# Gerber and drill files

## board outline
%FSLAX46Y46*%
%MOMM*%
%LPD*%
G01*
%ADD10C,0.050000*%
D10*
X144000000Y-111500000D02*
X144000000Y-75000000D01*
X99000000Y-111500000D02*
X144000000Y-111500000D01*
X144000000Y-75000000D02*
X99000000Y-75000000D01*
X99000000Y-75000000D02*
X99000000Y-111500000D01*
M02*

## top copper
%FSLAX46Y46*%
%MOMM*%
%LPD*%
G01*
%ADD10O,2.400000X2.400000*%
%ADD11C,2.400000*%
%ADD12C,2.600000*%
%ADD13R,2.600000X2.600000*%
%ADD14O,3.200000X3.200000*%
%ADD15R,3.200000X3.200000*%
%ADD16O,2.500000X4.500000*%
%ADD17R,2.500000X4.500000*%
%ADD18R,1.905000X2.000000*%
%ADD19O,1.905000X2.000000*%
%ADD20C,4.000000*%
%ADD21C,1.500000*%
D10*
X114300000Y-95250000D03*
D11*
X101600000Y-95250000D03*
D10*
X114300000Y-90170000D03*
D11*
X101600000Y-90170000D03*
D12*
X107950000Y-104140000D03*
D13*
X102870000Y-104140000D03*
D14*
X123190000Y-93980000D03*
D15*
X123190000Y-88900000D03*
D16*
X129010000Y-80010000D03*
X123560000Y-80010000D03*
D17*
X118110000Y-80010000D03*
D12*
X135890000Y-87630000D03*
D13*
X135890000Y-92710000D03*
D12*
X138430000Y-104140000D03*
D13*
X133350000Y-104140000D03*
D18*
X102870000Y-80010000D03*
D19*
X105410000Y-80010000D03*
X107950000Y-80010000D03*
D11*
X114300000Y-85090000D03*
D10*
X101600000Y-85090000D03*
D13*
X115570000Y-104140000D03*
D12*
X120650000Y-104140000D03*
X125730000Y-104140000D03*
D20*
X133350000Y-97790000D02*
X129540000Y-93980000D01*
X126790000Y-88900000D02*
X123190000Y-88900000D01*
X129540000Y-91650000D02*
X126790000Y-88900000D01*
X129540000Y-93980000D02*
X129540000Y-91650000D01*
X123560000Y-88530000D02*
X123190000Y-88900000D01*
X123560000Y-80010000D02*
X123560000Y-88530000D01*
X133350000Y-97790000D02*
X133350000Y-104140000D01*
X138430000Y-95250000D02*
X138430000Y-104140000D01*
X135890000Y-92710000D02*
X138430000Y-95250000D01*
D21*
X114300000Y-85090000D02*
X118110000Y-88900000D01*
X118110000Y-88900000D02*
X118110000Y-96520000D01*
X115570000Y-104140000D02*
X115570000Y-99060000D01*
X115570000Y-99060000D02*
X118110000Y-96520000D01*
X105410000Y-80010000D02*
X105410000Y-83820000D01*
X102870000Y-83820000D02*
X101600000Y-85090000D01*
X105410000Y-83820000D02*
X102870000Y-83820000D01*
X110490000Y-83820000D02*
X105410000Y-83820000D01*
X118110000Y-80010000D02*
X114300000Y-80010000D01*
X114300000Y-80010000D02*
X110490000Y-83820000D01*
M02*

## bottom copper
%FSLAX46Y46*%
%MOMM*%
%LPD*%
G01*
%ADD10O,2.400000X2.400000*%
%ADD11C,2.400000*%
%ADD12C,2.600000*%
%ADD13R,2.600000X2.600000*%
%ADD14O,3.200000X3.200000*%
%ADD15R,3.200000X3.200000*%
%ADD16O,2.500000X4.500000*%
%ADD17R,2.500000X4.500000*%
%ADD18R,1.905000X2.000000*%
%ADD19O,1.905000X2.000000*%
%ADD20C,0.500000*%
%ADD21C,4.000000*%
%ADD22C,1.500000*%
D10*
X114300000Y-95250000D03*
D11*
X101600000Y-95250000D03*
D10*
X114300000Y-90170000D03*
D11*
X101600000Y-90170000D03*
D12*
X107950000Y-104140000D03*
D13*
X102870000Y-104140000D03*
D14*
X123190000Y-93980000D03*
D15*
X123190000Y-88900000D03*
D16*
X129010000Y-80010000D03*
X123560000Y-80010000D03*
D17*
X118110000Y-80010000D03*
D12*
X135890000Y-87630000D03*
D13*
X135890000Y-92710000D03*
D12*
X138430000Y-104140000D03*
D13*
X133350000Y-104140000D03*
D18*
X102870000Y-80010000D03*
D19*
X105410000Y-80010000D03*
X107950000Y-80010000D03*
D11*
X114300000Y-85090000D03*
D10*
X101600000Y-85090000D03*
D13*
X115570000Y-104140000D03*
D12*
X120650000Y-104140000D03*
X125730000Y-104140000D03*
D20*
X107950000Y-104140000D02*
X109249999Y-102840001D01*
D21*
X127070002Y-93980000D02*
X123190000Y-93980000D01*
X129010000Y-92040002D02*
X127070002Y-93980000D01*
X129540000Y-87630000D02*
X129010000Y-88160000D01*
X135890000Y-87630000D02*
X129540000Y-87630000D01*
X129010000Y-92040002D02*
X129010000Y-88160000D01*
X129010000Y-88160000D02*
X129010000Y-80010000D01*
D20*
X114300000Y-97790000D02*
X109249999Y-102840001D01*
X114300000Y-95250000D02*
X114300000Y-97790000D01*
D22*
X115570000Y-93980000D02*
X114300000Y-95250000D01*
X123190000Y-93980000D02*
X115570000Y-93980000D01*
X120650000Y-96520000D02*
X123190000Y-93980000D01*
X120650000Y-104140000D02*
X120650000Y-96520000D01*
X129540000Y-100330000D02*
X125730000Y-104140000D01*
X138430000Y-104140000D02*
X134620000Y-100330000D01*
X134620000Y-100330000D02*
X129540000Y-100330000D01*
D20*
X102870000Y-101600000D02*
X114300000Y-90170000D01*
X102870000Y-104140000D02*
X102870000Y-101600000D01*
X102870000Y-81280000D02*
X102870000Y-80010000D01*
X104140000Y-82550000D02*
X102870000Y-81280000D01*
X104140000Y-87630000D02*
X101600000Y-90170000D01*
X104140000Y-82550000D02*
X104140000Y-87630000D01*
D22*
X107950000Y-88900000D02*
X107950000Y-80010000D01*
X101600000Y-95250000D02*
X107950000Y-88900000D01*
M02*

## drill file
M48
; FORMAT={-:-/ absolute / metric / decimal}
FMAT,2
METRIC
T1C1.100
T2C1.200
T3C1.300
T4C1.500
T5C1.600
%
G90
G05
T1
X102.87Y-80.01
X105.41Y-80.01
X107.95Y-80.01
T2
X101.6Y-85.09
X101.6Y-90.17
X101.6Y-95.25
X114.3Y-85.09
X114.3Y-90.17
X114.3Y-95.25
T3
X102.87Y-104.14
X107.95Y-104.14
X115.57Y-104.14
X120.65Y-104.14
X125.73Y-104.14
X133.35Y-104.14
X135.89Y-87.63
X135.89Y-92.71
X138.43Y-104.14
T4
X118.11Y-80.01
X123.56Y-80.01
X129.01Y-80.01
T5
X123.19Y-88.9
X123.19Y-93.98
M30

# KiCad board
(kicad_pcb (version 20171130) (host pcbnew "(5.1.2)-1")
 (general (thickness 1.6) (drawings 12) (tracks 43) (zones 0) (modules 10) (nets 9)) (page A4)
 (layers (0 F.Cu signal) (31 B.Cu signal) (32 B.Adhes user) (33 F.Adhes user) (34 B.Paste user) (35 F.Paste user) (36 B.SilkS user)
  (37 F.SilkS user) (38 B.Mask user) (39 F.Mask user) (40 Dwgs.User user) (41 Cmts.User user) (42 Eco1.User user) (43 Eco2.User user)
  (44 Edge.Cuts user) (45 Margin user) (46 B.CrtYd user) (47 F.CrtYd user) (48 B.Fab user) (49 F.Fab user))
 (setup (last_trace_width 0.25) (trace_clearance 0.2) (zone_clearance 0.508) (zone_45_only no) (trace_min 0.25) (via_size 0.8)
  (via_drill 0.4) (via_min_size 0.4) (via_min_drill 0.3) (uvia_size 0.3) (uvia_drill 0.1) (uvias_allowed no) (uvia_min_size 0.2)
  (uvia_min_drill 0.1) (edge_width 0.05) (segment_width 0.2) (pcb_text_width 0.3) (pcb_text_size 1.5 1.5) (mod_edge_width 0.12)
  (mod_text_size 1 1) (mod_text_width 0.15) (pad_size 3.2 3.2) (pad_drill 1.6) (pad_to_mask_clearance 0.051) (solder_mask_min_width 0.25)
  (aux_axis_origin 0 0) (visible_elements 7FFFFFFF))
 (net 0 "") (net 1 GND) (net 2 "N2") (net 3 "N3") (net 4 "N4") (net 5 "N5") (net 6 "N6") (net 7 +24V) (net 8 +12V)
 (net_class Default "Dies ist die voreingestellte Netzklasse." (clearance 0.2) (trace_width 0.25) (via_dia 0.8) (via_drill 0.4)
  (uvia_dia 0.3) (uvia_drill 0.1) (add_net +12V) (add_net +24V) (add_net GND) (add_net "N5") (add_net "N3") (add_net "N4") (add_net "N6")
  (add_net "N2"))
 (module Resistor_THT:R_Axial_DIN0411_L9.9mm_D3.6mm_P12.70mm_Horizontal (layer F.Cu) (at 101.6 95.25)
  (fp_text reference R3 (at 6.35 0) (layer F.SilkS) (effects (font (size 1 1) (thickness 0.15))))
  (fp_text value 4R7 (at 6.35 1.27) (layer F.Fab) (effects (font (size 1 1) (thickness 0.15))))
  (pad 2 thru_hole oval (at 12.7 0) (size 2.4 2.4) (drill 1.2) (layers *.Cu *.Mask) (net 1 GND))
  (pad 1 thru_hole circle (at 0 0) (size 2.4 2.4) (drill 1.2) (layers *.Cu *.Mask) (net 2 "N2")))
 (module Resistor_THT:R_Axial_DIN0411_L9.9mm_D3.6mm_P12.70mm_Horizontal (layer F.Cu) (at 101.6 90.17)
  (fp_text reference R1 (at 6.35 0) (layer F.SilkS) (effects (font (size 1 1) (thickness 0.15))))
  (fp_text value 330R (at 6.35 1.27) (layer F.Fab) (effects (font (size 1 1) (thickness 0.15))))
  (pad 2 thru_hole oval (at 12.7 0) (size 2.4 2.4) (drill 1.2) (layers *.Cu *.Mask) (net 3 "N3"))
  (pad 1 thru_hole circle (at 0 0) (size 2.4 2.4) (drill 1.2) (layers *.Cu *.Mask) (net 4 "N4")))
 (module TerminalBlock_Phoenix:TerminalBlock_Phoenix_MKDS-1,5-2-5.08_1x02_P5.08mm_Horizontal (layer F.Cu) (at 102.87 104.14)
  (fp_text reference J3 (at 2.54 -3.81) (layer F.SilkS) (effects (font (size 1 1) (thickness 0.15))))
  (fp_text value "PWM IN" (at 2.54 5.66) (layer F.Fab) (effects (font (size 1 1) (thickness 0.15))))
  (pad 2 thru_hole circle (at 5.08 0) (size 2.6 2.6) (drill 1.3) (layers *.Cu *.Mask) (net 1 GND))
  (pad 1 thru_hole rect (at 0 0) (size 2.6 2.6) (drill 1.3) (layers *.Cu *.Mask) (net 3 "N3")))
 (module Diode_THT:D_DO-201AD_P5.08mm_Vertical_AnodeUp (layer F.Cu) (at 123.19 88.9 270)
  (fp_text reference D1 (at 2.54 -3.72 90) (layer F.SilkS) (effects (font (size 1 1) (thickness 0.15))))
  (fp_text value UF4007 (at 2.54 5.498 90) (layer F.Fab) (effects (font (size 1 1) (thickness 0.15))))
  (pad 2 thru_hole oval (at 5.08 0 270) (size 3.2 3.2) (drill 1.6) (layers *.Cu *.Mask) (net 1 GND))
  (pad 1 thru_hole rect (at 0 0 270) (size 3.2 3.2) (drill 1.6) (layers *.Cu *.Mask) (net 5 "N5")))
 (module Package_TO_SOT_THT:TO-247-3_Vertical (layer F.Cu) (at 118.11 80.01)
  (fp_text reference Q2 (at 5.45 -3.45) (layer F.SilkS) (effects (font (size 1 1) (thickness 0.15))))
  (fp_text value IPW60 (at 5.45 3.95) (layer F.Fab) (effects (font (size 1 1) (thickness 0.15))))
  (pad 3 thru_hole oval (at 10.9 0) (size 2.5 4.5) (drill 1.5) (layers *.Cu *.Mask) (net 1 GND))
  (pad 2 thru_hole oval (at 5.45 0) (size 2.5 4.5) (drill 1.5) (layers *.Cu *.Mask) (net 5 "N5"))
  (pad 1 thru_hole rect (at 0 0) (size 2.5 4.5) (drill 1.5) (layers *.Cu *.Mask) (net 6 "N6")))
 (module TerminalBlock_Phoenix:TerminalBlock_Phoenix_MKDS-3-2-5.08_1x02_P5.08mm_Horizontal (layer F.Cu) (at 135.89 92.71 90)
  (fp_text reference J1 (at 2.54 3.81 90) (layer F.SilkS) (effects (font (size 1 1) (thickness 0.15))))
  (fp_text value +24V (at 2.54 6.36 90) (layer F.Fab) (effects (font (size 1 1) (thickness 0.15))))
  (pad 2 thru_hole circle (at 5.08 0 90) (size 2.6 2.6) (drill 1.3) (layers *.Cu *.Mask) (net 1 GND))
  (pad 1 thru_hole rect (at 0 0 90) (size 2.6 2.6) (drill 1.3) (layers *.Cu *.Mask) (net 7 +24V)))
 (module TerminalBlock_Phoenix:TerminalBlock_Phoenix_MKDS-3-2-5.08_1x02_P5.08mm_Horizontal (layer F.Cu) (at 133.35 104.14)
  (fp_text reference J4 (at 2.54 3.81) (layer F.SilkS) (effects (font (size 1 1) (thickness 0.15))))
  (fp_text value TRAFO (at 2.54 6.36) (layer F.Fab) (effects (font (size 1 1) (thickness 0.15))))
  (pad 2 thru_hole circle (at 5.08 0) (size 2.6 2.6) (drill 1.3) (layers *.Cu *.Mask) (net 7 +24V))
  (pad 1 thru_hole rect (at 0 0) (size 2.6 2.6) (drill 1.3) (layers *.Cu *.Mask) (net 5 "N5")))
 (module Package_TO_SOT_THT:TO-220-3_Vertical (layer F.Cu) (at 102.87 80.01)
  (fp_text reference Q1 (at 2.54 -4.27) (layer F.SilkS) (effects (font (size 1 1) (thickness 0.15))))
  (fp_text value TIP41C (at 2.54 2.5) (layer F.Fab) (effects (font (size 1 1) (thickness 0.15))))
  (pad 1 thru_hole rect (at 0 0) (size 1.905 2) (drill 1.1) (layers *.Cu *.Mask) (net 4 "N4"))
  (pad 2 thru_hole oval (at 2.54 0) (size 1.905 2) (drill 1.1) (layers *.Cu *.Mask) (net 6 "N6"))
  (pad 3 thru_hole oval (at 5.08 0) (size 1.905 2) (drill 1.1) (layers *.Cu *.Mask) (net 2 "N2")))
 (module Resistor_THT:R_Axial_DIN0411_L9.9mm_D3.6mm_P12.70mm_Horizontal (layer F.Cu) (at 114.3 85.09 180)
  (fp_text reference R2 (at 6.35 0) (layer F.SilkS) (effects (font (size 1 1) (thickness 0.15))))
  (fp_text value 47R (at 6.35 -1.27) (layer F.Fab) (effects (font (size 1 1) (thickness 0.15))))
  (pad 1 thru_hole circle (at 0 0 180) (size 2.4 2.4) (drill 1.2) (layers *.Cu *.Mask) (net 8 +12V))
  (pad 2 thru_hole oval (at 12.7 0 180) (size 2.4 2.4) (drill 1.2) (layers *.Cu *.Mask) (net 6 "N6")))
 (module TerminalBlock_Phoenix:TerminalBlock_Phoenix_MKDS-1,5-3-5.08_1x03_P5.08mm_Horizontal (layer F.Cu) (at 115.57 104.14)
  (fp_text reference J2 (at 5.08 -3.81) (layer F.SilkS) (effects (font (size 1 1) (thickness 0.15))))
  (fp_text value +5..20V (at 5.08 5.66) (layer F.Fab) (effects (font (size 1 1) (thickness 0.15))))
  (pad 1 thru_hole rect (at 0 0) (size 2.6 2.6) (drill 1.3) (layers *.Cu *.Mask) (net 8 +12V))
  (pad 2 thru_hole circle (at 5.08 0) (size 2.6 2.6) (drill 1.3) (layers *.Cu *.Mask) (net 1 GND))
  (pad 3 thru_hole circle (at 10.16 0) (size 2.6 2.6) (drill 1.3) (layers *.Cu *.Mask) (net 7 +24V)))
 (gr_line (start 144 111.5) (end 144 75) (layer Edge.Cuts) (width 0.05))
 (gr_line (start 99 111.5) (end 144 111.5) (layer Edge.Cuts) (width 0.05))
 (gr_line (start 144 75) (end 99 75) (layer Edge.Cuts) (width 0.05))
 (gr_line (start 99 75) (end 99 111.5) (layer Edge.Cuts) (width 0.05))
 (segment (start 133.35 97.79) (end 129.54 93.98) (width 4) (layer F.Cu) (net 5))
 (segment (start 126.79 88.9) (end 123.19 88.9) (width 4) (layer F.Cu) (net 5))
 (segment (start 129.54 91.65) (end 126.79 88.9) (width 4) (layer F.Cu) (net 5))
 (segment (start 129.54 93.98) (end 129.54 91.65) (width 4) (layer F.Cu) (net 5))
 (segment (start 123.56 88.53) (end 123.19 88.9) (width 4) (layer F.Cu) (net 5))
 (segment (start 123.56 80.01) (end 123.56 88.53) (width 4) (layer F.Cu) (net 5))
 (segment (start 133.35 97.79) (end 133.35 104.14) (width 4) (layer F.Cu) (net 5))
 (segment (start 107.95 104.14) (end 109.249999 102.840001) (width 0.5) (layer B.Cu) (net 1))
 (segment (start 127.070002 93.98) (end 123.19 93.98) (width 4) (layer B.Cu) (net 1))
 (segment (start 129.01 92.040002) (end 127.070002 93.98) (width 4) (layer B.Cu) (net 1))
 (segment (start 129.54 87.63) (end 129.01 88.16) (width 4) (layer B.Cu) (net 1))
 (segment (start 135.89 87.63) (end 129.54 87.63) (width 4) (layer B.Cu) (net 1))
 (segment (start 129.01 92.040002) (end 129.01 88.16) (width 4) (layer B.Cu) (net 1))
 (segment (start 129.01 88.16) (end 129.01 80.01) (width 4) (layer B.Cu) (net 1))
 (segment (start 114.3 97.79) (end 109.249999 102.840001) (width 0.5) (layer B.Cu) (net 1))
 (segment (start 114.3 95.25) (end 114.3 97.79) (width 0.5) (layer B.Cu) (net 1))
 (segment (start 115.57 93.98) (end 114.3 95.25) (width 1.5) (layer B.Cu) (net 1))
 (segment (start 123.19 93.98) (end 115.57 93.98) (width 1.5) (layer B.Cu) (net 1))
 (segment (start 120.65 96.52) (end 123.19 93.98) (width 1.5) (layer B.Cu) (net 1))
 (segment (start 120.65 104.14) (end 120.65 96.52) (width 1.5) (layer B.Cu) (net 1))
 (segment (start 138.43 95.25) (end 138.43 104.14) (width 4) (layer F.Cu) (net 7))
 (segment (start 135.89 92.71) (end 138.43 95.25) (width 4) (layer F.Cu) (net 7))
 (segment (start 129.54 100.33) (end 125.73 104.14) (width 1.5) (layer B.Cu) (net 7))
 (segment (start 138.43 104.14) (end 134.62 100.33) (width 1.5) (layer B.Cu) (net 7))
 (segment (start 134.62 100.33) (end 129.54 100.33) (width 1.5) (layer B.Cu) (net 7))
 (segment (start 114.3 85.09) (end 118.11 88.9) (width 1.5) (layer F.Cu) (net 8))
 (segment (start 118.11 88.9) (end 118.11 96.52) (width 1.5) (layer F.Cu) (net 8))
 (segment (start 115.57 104.14) (end 115.57 99.06) (width 1.5) (layer F.Cu) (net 8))
 (segment (start 115.57 99.06) (end 118.11 96.52) (width 1.5) (layer F.Cu) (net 8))
 (segment (start 102.87 101.6) (end 114.3 90.17) (width 0.5) (layer B.Cu) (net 3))
 (segment (start 102.87 104.14) (end 102.87 101.6) (width 0.5) (layer B.Cu) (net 3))
 (segment (start 102.87 81.28) (end 102.87 80.01) (width 0.5) (layer B.Cu) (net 4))
 (segment (start 104.14 82.55) (end 102.87 81.28) (width 0.5) (layer B.Cu) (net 4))
 (segment (start 104.14 87.63) (end 101.6 90.17) (width 0.5) (layer B.Cu) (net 4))
 (segment (start 104.14 82.55) (end 104.14 87.63) (width 0.5) (layer B.Cu) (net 4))
 (segment (start 105.41 80.01) (end 105.41 83.82) (width 1.5) (layer F.Cu) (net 6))
 (segment (start 102.87 83.82) (end 101.6 85.09) (width 1.5) (layer F.Cu) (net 6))
 (segment (start 105.41 83.82) (end 102.87 83.82) (width 1.5) (layer F.Cu) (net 6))
 (segment (start 110.49 83.82) (end 105.41 83.82) (width 1.5) (layer F.Cu) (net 6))
 (segment (start 118.11 80.01) (end 114.3 80.01) (width 1.5) (layer F.Cu) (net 6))
 (segment (start 114.3 80.01) (end 110.49 83.82) (width 1.5) (layer F.Cu) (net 6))
 (segment (start 107.95 88.9) (end 107.95 80.01) (width 1.5) (layer B.Cu) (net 2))
 (segment (start 101.6 95.25) (end 107.95 88.9) (width 1.5) (layer B.Cu) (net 2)))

